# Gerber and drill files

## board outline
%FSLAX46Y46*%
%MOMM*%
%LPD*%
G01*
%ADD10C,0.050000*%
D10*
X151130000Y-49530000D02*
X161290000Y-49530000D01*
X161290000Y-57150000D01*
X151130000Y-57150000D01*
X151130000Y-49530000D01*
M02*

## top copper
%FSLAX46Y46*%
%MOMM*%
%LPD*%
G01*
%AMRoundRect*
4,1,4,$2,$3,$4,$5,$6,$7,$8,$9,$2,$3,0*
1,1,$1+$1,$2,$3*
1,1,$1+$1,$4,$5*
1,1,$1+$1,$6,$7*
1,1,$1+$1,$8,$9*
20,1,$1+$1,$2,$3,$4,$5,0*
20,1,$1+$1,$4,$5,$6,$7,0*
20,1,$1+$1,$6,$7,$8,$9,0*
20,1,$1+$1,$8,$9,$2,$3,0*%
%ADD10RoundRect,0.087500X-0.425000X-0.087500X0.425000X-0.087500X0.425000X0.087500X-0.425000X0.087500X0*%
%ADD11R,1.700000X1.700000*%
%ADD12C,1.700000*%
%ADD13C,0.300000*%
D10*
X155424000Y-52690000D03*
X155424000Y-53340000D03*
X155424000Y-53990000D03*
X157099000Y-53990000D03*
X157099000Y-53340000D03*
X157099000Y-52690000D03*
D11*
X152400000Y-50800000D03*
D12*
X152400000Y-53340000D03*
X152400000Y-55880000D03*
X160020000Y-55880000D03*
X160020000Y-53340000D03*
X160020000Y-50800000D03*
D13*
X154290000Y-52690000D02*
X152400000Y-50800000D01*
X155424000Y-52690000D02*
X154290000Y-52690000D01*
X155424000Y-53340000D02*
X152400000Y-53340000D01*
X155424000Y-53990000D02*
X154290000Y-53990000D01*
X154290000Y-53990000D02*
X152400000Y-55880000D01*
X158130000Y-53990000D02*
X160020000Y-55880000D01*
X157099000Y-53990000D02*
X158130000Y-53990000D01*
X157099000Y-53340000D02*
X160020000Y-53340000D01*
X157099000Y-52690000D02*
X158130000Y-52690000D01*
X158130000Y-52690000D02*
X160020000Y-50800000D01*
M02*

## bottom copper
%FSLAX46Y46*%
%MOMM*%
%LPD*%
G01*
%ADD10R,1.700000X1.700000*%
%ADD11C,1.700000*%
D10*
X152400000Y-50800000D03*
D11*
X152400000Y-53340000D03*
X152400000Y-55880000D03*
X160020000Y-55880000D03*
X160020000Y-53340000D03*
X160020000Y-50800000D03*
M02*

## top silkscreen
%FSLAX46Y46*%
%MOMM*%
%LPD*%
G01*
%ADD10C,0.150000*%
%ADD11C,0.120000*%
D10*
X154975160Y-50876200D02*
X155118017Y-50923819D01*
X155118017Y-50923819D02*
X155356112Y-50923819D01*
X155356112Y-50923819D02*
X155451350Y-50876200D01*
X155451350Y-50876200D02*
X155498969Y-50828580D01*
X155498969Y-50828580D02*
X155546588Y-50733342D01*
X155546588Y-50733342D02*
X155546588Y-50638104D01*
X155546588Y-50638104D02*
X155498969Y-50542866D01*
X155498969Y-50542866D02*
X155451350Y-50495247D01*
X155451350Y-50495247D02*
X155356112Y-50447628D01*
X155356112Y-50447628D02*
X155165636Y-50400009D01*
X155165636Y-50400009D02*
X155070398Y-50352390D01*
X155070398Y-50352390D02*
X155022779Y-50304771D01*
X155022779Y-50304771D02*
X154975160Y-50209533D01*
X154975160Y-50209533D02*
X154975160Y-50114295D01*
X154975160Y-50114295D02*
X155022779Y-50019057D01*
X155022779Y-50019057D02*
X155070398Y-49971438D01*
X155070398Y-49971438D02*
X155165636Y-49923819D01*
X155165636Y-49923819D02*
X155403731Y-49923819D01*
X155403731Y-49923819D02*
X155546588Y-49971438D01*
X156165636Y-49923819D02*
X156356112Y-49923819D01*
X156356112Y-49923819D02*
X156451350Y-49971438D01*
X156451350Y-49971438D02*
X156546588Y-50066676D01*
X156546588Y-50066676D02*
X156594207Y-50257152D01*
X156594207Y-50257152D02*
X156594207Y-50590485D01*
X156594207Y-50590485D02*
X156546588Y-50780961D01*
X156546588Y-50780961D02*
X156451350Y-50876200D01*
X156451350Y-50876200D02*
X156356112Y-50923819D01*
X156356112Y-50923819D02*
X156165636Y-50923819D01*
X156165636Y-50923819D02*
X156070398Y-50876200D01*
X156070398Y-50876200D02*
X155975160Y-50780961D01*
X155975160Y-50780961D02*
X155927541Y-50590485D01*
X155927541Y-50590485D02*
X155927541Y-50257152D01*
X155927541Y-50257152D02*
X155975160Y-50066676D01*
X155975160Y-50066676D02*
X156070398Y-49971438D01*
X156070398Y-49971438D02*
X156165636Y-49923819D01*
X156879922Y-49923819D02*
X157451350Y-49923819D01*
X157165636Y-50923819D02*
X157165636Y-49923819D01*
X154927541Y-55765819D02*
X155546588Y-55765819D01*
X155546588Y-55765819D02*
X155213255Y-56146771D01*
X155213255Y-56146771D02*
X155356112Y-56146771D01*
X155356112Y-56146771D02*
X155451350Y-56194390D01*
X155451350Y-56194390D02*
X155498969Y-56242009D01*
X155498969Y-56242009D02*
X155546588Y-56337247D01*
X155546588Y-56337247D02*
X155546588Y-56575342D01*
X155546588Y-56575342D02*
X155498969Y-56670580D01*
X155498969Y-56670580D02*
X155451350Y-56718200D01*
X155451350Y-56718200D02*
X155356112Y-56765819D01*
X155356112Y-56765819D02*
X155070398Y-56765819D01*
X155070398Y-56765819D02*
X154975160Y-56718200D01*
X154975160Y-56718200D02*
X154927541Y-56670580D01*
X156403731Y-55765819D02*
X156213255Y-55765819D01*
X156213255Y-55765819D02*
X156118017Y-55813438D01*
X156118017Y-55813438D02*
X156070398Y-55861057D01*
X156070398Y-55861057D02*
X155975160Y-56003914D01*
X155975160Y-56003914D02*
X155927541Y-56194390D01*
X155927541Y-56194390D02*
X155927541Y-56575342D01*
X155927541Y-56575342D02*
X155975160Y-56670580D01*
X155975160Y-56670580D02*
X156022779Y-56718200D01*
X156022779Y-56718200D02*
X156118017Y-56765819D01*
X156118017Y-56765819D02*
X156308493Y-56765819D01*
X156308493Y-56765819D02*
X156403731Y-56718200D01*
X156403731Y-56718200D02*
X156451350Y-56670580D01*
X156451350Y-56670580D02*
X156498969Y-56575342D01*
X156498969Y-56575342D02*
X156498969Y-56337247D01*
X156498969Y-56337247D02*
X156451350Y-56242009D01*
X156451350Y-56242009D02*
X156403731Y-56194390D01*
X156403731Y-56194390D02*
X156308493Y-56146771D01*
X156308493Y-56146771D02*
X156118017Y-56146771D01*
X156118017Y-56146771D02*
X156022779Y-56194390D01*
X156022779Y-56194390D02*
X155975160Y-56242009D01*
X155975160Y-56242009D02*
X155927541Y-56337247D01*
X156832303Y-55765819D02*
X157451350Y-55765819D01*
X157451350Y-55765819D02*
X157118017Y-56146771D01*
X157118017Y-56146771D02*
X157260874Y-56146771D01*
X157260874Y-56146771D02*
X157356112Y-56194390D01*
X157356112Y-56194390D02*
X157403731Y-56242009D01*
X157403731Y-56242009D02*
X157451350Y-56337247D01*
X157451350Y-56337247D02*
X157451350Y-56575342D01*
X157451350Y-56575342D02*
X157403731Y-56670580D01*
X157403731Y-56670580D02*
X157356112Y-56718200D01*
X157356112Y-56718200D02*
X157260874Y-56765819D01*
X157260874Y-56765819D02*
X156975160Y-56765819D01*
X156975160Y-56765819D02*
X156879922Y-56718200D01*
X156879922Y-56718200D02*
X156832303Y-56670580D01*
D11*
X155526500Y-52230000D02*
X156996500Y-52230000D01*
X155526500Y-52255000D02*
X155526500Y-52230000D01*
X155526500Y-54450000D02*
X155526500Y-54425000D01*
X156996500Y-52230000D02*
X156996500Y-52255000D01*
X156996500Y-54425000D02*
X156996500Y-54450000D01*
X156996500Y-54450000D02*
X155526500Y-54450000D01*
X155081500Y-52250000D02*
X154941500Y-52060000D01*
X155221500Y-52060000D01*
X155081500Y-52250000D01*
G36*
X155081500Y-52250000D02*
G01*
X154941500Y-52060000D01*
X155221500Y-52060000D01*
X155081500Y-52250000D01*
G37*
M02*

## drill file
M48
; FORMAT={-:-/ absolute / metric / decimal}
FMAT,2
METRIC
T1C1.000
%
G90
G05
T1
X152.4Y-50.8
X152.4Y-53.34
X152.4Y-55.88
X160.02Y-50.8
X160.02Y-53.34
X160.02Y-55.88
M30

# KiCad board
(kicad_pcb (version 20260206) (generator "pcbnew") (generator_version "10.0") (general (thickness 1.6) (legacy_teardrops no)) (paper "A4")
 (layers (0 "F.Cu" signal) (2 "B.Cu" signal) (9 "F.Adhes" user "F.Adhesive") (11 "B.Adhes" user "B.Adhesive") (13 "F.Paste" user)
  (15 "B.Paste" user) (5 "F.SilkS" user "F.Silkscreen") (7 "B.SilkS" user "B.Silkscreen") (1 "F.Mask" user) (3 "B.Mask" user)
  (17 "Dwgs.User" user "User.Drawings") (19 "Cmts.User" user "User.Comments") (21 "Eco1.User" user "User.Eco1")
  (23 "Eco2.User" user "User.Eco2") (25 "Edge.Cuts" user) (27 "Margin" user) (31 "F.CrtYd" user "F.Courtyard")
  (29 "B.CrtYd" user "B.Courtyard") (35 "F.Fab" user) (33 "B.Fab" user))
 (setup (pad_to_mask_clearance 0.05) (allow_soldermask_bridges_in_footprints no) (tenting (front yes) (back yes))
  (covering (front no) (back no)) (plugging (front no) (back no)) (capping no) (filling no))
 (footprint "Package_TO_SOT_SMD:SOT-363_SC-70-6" (layer "F.Cu") (at 156.2615 53.34)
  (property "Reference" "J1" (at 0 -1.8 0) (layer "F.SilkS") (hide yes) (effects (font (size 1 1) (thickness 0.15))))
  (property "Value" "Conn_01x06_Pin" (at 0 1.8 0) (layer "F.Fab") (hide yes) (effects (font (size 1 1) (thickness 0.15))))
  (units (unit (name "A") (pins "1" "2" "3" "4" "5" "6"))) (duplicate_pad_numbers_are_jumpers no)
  (fp_line (start -0.735 -1.11) (end 0.735 -1.11) (stroke (width 0.12) (type solid)) (layer "F.SilkS"))
  (fp_line (start -0.735 -1.085) (end -0.735 -1.11) (stroke (width 0.12) (type solid)) (layer "F.SilkS"))
  (fp_line (start -0.735 1.11) (end -0.735 1.085) (stroke (width 0.12) (type solid)) (layer "F.SilkS"))
  (fp_line (start 0.735 -1.11) (end 0.735 -1.085) (stroke (width 0.12) (type solid)) (layer "F.SilkS"))
  (fp_line (start 0.735 1.085) (end 0.735 1.11) (stroke (width 0.12) (type solid)) (layer "F.SilkS"))
  (fp_line (start 0.735 1.11) (end -0.735 1.11) (stroke (width 0.12) (type solid)) (layer "F.SilkS"))
  (fp_poly (pts (xy -1.18 -1.09) (xy -1.32 -1.28) (xy -1.04 -1.28)) (stroke (width 0.12) (type solid)) (fill yes) (layer "F.SilkS"))
  (pad "1" smd roundrect (at -0.8375 -0.65) (size 1.025 0.35) (layers "F.Cu" "F.Mask" "F.Paste") (roundrect_rratio 0.25)
   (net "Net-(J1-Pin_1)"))
  (pad "2" smd roundrect (at -0.8375 0) (size 1.025 0.35) (layers "F.Cu" "F.Mask" "F.Paste") (roundrect_rratio 0.25) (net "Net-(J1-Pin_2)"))
  (pad "3" smd roundrect (at -0.8375 0.65) (size 1.025 0.35) (layers "F.Cu" "F.Mask" "F.Paste") (roundrect_rratio 0.25)
   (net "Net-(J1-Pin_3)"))
  (pad "4" smd roundrect (at 0.8375 0.65) (size 1.025 0.35) (layers "F.Cu" "F.Mask" "F.Paste") (roundrect_rratio 0.25)
   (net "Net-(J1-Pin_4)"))
  (pad "5" smd roundrect (at 0.8375 0) (size 1.025 0.35) (layers "F.Cu" "F.Mask" "F.Paste") (roundrect_rratio 0.25) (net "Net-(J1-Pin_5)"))
  (pad "6" smd roundrect (at 0.8375 -0.65) (size 1.025 0.35) (layers "F.Cu" "F.Mask" "F.Paste") (roundrect_rratio 0.25)
   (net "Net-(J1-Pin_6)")))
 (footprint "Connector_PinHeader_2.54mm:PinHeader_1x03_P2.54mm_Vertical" (layer "B.Cu") (at 152.4 50.8 180)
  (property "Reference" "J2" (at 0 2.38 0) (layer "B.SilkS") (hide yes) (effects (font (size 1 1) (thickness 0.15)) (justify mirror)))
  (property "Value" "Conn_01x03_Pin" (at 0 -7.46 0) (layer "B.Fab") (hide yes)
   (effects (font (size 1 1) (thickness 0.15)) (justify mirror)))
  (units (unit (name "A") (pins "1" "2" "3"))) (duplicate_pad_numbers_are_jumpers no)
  (pad "1" thru_hole rect (at 0 0 180) (size 1.7 1.7) (drill 1) (layers "*.Cu" "*.Mask") (remove_unused_layers no) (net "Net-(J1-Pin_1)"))
  (pad "2" thru_hole circle (at 0 -2.54 180) (size 1.7 1.7) (drill 1) (layers "*.Cu" "*.Mask") (remove_unused_layers no)
   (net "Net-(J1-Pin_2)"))
  (pad "3" thru_hole circle (at 0 -5.08 180) (size 1.7 1.7) (drill 1) (layers "*.Cu" "*.Mask") (remove_unused_layers no)
   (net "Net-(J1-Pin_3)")))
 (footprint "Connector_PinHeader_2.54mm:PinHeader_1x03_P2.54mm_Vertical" (layer "B.Cu") (at 160.02 55.88)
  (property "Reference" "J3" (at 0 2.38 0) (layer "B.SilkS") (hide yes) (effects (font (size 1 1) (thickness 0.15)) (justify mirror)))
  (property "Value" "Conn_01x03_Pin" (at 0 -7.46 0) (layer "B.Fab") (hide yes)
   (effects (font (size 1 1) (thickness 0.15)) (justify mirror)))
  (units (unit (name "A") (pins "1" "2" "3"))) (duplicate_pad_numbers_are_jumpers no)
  (pad "1" thru_hole circle (at 0 0) (size 1.7 1.7) (drill 1) (layers "*.Cu" "*.Mask") (remove_unused_layers no) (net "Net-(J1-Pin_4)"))
  (pad "2" thru_hole circle (at 0 -2.54) (size 1.7 1.7) (drill 1) (layers "*.Cu" "*.Mask") (remove_unused_layers no) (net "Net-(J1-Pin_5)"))
  (pad "3" thru_hole circle (at 0 -5.08) (size 1.7 1.7) (drill 1) (layers "*.Cu" "*.Mask") (remove_unused_layers no) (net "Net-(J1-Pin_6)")))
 (gr_rect (start 151.13 49.53) (end 161.29 57.15) (stroke (width 0.05) (type default)) (fill no) (layer "Edge.Cuts"))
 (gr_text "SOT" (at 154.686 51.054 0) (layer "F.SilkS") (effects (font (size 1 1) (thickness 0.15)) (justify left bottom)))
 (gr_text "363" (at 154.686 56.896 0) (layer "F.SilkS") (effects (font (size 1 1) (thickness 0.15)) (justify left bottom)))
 (segment (start 154.29 52.69) (end 152.4 50.8) (width 0.3) (layer "F.Cu") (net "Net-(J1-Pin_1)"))
 (segment (start 155.424 52.69) (end 154.29 52.69) (width 0.3) (layer "F.Cu") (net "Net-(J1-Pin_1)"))
 (segment (start 155.424 53.34) (end 152.4 53.34) (width 0.3) (layer "F.Cu") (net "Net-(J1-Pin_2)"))
 (segment (start 155.424 53.99) (end 154.29 53.99) (width 0.3) (layer "F.Cu") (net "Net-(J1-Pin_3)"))
 (segment (start 154.29 53.99) (end 152.4 55.88) (width 0.3) (layer "F.Cu") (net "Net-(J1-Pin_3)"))
 (segment (start 158.13 53.99) (end 160.02 55.88) (width 0.3) (layer "F.Cu") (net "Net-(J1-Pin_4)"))
 (segment (start 157.099 53.99) (end 158.13 53.99) (width 0.3) (layer "F.Cu") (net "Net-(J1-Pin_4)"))
 (segment (start 157.099 53.34) (end 160.02 53.34) (width 0.3) (layer "F.Cu") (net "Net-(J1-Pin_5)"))
 (segment (start 157.099 52.69) (end 158.13 52.69) (width 0.3) (layer "F.Cu") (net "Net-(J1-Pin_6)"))
 (segment (start 158.13 52.69) (end 160.02 50.8) (width 0.3) (layer "F.Cu") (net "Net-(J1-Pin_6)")))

